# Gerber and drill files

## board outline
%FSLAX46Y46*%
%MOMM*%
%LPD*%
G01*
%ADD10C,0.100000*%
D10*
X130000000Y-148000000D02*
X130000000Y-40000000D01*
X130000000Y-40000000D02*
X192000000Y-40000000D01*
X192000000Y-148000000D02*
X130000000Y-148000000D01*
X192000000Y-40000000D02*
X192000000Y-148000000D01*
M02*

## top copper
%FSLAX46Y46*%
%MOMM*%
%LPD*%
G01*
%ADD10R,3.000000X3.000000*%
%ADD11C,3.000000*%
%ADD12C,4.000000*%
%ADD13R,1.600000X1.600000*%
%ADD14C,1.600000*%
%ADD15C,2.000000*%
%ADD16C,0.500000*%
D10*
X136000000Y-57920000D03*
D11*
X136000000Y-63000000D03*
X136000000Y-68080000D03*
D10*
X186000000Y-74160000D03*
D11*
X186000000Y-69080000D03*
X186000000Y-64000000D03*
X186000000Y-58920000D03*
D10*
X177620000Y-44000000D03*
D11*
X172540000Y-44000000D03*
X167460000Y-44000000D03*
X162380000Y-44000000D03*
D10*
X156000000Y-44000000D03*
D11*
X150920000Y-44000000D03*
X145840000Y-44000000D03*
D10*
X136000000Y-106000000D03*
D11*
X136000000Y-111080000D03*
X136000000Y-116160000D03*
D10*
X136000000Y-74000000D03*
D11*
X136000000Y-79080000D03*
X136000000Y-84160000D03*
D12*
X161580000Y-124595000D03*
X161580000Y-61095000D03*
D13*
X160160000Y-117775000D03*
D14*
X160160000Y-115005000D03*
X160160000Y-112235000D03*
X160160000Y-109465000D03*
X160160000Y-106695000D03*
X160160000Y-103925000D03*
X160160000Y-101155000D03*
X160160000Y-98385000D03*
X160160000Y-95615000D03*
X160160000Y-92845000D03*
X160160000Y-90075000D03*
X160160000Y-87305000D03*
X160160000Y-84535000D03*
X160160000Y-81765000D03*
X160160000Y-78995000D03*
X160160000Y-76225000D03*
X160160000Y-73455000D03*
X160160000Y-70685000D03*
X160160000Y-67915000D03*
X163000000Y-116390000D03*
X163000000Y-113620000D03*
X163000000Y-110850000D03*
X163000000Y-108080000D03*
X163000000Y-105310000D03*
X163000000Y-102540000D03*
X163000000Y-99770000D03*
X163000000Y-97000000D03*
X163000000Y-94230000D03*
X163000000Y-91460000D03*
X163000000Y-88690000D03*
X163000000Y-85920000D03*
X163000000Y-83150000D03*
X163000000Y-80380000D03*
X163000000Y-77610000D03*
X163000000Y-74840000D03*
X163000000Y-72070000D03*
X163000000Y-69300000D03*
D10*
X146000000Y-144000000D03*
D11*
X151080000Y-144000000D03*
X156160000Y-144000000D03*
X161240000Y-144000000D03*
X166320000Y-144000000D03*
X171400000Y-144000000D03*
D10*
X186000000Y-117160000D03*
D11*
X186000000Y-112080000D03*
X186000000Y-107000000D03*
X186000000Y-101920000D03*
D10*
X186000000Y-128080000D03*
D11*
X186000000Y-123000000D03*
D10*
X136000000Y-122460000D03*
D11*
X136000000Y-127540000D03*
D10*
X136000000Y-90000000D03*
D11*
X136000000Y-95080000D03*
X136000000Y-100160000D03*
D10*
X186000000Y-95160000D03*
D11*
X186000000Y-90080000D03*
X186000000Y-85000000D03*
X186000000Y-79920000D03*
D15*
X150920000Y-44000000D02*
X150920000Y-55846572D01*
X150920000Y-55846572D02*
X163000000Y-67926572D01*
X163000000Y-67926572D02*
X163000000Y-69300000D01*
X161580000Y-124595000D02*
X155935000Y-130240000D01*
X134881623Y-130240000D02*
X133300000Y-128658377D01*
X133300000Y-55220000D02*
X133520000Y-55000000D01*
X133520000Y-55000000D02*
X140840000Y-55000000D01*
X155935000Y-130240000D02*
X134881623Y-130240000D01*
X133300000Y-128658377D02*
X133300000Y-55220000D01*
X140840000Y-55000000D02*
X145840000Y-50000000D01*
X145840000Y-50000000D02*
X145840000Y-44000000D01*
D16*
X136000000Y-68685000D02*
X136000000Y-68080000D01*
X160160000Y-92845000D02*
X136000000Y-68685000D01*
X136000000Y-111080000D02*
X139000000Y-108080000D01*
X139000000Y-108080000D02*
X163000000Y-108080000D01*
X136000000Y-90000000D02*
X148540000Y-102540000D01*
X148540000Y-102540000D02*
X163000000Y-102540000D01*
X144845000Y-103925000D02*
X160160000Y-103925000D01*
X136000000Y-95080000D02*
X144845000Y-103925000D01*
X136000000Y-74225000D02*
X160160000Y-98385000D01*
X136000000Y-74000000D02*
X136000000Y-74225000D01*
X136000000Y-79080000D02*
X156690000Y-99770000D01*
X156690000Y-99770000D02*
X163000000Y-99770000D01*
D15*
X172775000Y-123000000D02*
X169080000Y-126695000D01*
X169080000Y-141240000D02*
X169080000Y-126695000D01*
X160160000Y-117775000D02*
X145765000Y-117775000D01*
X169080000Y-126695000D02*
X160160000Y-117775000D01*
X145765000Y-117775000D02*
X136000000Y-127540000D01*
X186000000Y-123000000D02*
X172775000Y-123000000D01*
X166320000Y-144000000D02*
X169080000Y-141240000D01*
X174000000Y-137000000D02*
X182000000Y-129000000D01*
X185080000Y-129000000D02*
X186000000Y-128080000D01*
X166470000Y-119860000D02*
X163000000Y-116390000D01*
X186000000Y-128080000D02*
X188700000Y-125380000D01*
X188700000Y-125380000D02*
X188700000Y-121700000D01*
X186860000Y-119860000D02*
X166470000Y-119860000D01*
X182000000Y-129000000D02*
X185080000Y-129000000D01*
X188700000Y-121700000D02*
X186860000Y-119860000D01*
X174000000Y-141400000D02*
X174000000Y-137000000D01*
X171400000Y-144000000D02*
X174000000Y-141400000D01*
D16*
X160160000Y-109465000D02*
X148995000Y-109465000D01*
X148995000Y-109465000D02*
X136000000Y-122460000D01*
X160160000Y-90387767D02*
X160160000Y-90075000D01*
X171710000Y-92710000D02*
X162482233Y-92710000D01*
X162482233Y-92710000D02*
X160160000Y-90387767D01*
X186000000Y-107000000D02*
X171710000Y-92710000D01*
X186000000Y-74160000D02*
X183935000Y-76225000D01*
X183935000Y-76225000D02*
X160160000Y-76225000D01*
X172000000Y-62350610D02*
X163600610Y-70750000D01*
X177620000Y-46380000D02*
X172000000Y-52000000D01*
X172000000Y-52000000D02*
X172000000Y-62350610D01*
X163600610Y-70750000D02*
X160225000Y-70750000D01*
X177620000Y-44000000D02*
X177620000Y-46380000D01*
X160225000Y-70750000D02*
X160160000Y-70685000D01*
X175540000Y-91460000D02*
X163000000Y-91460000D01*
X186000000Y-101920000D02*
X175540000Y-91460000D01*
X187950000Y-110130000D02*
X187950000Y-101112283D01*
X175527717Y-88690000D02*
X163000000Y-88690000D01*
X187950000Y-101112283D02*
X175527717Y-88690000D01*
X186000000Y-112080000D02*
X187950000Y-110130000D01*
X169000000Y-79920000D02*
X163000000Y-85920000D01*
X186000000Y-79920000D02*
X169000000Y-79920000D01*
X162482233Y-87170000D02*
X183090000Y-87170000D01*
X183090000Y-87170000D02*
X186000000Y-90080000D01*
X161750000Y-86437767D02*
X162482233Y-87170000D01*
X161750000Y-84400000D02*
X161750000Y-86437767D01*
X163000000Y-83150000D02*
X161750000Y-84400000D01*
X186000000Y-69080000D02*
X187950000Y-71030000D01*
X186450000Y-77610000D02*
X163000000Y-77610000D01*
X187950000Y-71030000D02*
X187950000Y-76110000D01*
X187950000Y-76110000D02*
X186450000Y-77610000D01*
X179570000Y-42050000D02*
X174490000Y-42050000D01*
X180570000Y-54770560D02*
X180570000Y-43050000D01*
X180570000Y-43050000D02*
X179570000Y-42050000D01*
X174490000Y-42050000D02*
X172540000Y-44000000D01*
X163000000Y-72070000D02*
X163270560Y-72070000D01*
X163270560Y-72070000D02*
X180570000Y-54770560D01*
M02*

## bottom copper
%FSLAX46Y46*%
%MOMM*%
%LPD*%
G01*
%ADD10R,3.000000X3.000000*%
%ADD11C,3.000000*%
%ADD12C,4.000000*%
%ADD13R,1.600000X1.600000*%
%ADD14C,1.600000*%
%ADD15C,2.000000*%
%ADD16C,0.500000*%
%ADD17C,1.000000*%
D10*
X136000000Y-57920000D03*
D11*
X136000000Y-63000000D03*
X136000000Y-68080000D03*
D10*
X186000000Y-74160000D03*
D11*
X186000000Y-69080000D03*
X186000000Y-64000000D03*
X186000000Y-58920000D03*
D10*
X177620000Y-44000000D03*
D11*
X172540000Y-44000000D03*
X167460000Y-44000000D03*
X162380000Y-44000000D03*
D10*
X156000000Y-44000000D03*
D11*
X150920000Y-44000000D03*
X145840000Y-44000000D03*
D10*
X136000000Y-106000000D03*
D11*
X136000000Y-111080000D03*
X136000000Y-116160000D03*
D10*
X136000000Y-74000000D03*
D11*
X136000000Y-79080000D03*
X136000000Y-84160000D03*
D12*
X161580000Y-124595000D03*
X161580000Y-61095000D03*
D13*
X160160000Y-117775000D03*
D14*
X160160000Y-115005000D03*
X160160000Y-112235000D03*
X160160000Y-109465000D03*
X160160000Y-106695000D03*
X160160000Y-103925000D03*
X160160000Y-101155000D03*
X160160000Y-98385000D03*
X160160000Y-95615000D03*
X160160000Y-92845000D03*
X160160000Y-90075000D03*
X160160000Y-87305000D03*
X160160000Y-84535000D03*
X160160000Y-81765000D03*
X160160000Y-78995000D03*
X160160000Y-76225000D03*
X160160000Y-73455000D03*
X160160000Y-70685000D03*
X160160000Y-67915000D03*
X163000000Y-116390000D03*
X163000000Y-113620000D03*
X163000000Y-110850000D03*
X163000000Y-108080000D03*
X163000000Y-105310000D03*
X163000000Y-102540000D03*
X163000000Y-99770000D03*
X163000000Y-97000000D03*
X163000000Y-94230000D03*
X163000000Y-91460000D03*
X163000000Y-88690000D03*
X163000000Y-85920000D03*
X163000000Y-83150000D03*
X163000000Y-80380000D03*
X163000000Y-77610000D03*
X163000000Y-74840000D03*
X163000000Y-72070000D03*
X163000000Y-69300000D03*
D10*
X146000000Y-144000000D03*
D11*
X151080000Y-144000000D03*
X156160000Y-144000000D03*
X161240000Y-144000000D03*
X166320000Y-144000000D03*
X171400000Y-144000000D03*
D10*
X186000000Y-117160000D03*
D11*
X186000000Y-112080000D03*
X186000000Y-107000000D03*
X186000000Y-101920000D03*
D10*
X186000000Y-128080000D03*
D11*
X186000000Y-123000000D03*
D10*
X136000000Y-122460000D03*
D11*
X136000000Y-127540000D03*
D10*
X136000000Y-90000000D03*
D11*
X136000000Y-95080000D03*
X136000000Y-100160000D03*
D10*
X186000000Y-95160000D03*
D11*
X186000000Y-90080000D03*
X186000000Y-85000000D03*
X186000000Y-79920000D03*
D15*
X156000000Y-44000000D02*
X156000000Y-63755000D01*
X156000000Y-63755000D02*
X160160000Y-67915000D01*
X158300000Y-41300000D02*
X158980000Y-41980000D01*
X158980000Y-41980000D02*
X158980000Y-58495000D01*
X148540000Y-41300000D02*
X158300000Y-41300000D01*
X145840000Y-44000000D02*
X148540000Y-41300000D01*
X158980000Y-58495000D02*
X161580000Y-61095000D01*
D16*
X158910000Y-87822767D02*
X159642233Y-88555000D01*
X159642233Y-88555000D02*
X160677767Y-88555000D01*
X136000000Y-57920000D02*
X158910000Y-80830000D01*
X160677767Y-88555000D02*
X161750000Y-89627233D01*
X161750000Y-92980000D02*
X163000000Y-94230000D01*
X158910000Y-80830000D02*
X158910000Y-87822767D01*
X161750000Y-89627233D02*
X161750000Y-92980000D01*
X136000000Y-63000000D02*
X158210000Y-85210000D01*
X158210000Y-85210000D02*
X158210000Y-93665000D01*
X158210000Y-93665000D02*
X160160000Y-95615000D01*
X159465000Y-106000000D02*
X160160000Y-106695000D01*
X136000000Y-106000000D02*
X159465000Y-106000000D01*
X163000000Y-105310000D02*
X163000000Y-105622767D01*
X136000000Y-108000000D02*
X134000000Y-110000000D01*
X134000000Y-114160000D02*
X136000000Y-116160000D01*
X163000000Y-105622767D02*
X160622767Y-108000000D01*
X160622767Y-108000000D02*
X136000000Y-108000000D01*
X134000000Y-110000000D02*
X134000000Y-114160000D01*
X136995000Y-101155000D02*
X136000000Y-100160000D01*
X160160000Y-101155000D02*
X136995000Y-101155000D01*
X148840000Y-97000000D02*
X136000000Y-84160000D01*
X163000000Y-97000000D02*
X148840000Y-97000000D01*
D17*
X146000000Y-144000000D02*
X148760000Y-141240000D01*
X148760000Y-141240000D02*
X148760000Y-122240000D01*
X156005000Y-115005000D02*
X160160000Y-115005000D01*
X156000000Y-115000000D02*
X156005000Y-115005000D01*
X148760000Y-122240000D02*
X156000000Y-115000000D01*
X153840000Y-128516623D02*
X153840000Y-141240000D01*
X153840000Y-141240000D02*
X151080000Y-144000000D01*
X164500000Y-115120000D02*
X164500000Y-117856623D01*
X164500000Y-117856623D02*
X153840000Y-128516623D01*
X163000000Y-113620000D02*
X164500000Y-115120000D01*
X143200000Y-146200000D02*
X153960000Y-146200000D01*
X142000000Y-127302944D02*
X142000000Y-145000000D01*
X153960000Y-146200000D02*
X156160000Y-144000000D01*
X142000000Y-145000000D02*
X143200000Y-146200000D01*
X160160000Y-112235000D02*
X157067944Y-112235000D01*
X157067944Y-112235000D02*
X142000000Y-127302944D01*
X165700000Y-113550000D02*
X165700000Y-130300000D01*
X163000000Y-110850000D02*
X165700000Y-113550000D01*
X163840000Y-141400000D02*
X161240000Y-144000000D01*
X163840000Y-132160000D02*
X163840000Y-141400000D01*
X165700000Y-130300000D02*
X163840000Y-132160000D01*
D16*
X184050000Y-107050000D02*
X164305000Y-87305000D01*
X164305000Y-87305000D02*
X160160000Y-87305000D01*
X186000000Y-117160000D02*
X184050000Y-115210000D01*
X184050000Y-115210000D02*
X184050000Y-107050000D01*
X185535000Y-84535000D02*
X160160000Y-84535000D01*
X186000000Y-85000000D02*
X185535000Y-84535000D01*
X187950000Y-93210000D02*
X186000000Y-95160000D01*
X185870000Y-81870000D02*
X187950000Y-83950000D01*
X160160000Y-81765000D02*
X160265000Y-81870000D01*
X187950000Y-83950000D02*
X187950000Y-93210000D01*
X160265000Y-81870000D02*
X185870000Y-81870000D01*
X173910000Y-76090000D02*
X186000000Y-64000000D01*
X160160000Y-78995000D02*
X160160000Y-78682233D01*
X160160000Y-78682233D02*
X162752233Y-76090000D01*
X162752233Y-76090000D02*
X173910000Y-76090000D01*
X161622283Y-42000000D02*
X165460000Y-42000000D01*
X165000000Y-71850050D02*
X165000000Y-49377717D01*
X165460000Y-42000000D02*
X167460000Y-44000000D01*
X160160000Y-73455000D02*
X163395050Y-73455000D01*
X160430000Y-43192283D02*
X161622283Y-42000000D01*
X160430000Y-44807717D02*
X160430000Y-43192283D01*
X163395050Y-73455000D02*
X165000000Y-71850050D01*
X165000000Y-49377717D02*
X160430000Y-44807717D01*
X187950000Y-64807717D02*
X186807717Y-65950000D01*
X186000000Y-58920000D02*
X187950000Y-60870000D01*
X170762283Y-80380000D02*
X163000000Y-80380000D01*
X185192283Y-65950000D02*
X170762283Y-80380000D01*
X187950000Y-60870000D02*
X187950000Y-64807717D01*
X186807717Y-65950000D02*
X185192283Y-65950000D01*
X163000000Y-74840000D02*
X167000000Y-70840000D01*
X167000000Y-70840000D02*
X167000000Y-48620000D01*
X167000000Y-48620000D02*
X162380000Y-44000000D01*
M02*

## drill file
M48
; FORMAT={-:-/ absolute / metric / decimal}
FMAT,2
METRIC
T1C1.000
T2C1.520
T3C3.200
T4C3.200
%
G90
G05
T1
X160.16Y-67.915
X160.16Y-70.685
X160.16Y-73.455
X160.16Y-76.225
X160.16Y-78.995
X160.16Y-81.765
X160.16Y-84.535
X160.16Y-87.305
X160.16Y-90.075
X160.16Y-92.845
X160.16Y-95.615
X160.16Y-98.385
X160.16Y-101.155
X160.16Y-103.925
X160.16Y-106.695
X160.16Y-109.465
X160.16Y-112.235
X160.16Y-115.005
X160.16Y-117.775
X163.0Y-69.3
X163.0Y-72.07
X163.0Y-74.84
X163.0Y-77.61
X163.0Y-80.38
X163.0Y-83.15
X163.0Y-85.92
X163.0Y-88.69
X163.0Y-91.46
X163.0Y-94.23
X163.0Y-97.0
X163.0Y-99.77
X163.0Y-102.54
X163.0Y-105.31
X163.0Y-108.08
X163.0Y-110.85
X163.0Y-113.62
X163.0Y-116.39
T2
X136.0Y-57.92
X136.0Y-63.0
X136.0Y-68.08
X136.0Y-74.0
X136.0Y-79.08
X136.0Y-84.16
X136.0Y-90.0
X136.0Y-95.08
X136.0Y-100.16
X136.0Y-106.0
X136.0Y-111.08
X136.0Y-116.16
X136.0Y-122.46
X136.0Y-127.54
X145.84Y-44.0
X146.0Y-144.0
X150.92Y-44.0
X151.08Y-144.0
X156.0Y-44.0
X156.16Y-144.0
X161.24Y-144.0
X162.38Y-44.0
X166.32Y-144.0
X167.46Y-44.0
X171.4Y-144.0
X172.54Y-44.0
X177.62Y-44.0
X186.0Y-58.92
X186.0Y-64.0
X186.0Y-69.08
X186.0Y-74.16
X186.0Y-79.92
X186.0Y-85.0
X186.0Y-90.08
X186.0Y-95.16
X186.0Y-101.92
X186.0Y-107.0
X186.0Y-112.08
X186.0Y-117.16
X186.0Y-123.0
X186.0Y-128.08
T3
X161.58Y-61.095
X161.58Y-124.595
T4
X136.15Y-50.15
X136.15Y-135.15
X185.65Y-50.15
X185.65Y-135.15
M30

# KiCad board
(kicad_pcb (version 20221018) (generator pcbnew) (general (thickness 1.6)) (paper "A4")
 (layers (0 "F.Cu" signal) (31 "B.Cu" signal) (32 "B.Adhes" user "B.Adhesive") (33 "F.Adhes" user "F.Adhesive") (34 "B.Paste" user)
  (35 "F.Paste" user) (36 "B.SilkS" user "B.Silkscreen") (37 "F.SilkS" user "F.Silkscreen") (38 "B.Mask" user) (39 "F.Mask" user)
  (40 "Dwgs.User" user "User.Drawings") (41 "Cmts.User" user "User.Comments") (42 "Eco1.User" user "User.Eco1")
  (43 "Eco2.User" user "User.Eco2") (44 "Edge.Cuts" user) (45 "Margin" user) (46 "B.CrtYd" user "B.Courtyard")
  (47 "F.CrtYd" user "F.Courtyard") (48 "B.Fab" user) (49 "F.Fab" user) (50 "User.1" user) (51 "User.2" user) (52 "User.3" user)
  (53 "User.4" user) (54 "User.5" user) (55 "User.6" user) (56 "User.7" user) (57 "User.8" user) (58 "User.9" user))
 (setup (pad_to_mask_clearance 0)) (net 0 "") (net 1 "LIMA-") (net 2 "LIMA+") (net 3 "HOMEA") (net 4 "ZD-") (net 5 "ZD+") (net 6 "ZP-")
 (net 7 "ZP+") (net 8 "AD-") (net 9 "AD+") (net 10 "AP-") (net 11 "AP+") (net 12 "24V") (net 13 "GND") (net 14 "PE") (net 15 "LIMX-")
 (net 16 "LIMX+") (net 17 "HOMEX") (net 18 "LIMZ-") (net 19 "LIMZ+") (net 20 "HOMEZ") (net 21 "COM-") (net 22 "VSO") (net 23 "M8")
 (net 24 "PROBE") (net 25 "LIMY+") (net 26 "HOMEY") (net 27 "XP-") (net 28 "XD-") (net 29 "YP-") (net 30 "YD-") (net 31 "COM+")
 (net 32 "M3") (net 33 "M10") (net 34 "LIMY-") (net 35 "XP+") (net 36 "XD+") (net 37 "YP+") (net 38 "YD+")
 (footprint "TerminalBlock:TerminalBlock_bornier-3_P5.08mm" (layer "F.Cu") (at 136 57.92 -90)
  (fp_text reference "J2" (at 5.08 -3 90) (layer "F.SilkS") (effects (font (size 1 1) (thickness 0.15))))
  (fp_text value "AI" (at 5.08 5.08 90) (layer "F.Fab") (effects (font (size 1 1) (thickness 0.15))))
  (pad "1" thru_hole rect (at 0 0 270) (size 3 3) (drill 1.52) (layers "*.Cu" "*.Mask") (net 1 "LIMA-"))
  (pad "2" thru_hole circle (at 5.08 0 270) (size 3 3) (drill 1.52) (layers "*.Cu" "*.Mask") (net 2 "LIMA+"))
  (pad "3" thru_hole circle (at 10.16 0 270) (size 3 3) (drill 1.52) (layers "*.Cu" "*.Mask") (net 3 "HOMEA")))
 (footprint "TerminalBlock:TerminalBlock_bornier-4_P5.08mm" (layer "F.Cu") (at 186 74.16 90)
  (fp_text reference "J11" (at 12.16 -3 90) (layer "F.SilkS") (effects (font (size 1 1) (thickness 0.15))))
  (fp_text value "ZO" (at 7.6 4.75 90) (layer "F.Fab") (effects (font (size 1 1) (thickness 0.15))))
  (pad "1" thru_hole rect (at 0 0 90) (size 3 3) (drill 1.52) (layers "*.Cu" "*.Mask") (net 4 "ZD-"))
  (pad "2" thru_hole circle (at 5.08 0 90) (size 3 3) (drill 1.52) (layers "*.Cu" "*.Mask") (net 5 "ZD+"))
  (pad "3" thru_hole circle (at 10.16 0 90) (size 3 3) (drill 1.52) (layers "*.Cu" "*.Mask") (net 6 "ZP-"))
  (pad "4" thru_hole circle (at 15.24 0 90) (size 3 3) (drill 1.52) (layers "*.Cu" "*.Mask") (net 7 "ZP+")))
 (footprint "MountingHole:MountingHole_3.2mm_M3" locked (layer "F.Cu") (at 185.65 50.15)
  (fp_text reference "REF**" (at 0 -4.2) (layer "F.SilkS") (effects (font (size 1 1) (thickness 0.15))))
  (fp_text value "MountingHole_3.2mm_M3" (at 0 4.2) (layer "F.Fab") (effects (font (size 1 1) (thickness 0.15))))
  (pad "" np_thru_hole circle locked (at 0 0) (size 3.2 3.2) (drill 3.2) (layers "*.Cu" "*.Mask")))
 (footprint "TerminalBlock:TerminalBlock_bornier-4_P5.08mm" (layer "F.Cu") (at 177.62 44 180)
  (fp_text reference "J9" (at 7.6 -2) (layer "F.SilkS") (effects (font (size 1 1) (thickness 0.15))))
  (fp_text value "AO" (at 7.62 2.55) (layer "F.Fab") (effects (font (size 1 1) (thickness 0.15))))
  (pad "1" thru_hole rect (at 0 0 180) (size 3 3) (drill 1.52) (layers "*.Cu" "*.Mask") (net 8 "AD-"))
  (pad "2" thru_hole circle (at 5.08 0 180) (size 3 3) (drill 1.52) (layers "*.Cu" "*.Mask") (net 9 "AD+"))
  (pad "3" thru_hole circle (at 10.16 0 180) (size 3 3) (drill 1.52) (layers "*.Cu" "*.Mask") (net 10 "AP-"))
  (pad "4" thru_hole circle (at 15.24 0 180) (size 3 3) (drill 1.52) (layers "*.Cu" "*.Mask") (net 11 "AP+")))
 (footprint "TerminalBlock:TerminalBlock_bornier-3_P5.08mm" (layer "F.Cu") (at 156 44 180)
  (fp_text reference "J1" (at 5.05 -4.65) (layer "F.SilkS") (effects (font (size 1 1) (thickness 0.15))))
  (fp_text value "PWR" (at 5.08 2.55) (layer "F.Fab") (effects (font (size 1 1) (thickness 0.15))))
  (pad "1" thru_hole rect (at 0 0 180) (size 3 3) (drill 1.52) (layers "*.Cu" "*.Mask") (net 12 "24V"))
  (pad "2" thru_hole circle (at 5.08 0 180) (size 3 3) (drill 1.52) (layers "*.Cu" "*.Mask") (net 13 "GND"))
  (pad "3" thru_hole circle (at 10.16 0 180) (size 3 3) (drill 1.52) (layers "*.Cu" "*.Mask") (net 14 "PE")))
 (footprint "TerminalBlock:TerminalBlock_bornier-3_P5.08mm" (layer "F.Cu") (at 136 106 -90)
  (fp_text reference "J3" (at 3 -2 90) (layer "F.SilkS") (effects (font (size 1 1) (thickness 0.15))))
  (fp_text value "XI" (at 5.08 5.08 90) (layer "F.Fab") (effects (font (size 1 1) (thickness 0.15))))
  (pad "1" thru_hole rect (at 0 0 270) (size 3 3) (drill 1.52) (layers "*.Cu" "*.Mask") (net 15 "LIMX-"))
  (pad "2" thru_hole circle (at 5.08 0 270) (size 3 3) (drill 1.52) (layers "*.Cu" "*.Mask") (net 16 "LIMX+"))
  (pad "3" thru_hole circle (at 10.16 0 270) (size 3 3) (drill 1.52) (layers "*.Cu" "*.Mask") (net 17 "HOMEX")))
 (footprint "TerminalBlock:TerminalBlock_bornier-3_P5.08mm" (layer "F.Cu") (at 136 74 -90)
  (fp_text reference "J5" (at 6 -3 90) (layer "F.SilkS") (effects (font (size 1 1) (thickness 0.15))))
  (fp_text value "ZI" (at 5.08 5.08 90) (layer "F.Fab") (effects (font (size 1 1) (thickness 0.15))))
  (pad "1" thru_hole rect (at 0 0 270) (size 3 3) (drill 1.52) (layers "*.Cu" "*.Mask") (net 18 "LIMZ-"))
  (pad "2" thru_hole circle (at 5.08 0 270) (size 3 3) (drill 1.52) (layers "*.Cu" "*.Mask") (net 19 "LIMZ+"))
  (pad "3" thru_hole circle (at 10.16 0 270) (size 3 3) (drill 1.52) (layers "*.Cu" "*.Mask") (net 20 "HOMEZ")))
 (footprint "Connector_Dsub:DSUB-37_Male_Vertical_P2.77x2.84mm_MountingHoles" (layer "F.Cu") (at 160.16 117.775 90)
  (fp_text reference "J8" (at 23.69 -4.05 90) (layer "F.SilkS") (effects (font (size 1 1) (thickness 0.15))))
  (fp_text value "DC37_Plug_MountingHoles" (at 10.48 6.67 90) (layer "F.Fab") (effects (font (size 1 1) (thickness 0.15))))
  (pad "0" thru_hole circle (at -6.82 1.42 90) (size 4 4) (drill 3.2) (layers "*.Cu" "*.Mask") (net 14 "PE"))
  (pad "0" thru_hole circle (at 56.68 1.42 90) (size 4 4) (drill 3.2) (layers "*.Cu" "*.Mask") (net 14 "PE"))
  (pad "1" thru_hole rect (at 0 0 90) (size 1.6 1.6) (drill 1) (layers "*.Cu" "*.Mask") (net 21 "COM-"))
  (pad "2" thru_hole circle (at 2.77 0 90) (size 1.6 1.6) (drill 1) (layers "*.Cu" "*.Mask") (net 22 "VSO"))
  (pad "3" thru_hole circle (at 5.54 0 90) (size 1.6 1.6) (drill 1) (layers "*.Cu" "*.Mask") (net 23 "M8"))
  (pad "4" thru_hole circle (at 8.31 0 90) (size 1.6 1.6) (drill 1) (layers "*.Cu" "*.Mask") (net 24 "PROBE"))
  (pad "5" thru_hole circle (at 11.08 0 90) (size 1.6 1.6) (drill 1) (layers "*.Cu" "*.Mask") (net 15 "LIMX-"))
  (pad "6" thru_hole circle (at 13.85 0 90) (size 1.6 1.6) (drill 1) (layers "*.Cu" "*.Mask") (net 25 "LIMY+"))
  (pad "7" thru_hole circle (at 16.62 0 90) (size 1.6 1.6) (drill 1) (layers "*.Cu" "*.Mask") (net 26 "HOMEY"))
  (pad "8" thru_hole circle (at 19.39 0 90) (size 1.6 1.6) (drill 1) (layers "*.Cu" "*.Mask") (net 18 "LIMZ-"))
  (pad "9" thru_hole circle (at 22.16 0 90) (size 1.6 1.6) (drill 1) (layers "*.Cu" "*.Mask") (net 2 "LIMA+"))
  (pad "10" thru_hole circle (at 24.93 0 90) (size 1.6 1.6) (drill 1) (layers "*.Cu" "*.Mask") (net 3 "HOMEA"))
  (pad "11" thru_hole circle (at 27.7 0 90) (size 1.6 1.6) (drill 1) (layers "*.Cu" "*.Mask") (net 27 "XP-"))
  (pad "12" thru_hole circle (at 30.47 0 90) (size 1.6 1.6) (drill 1) (layers "*.Cu" "*.Mask") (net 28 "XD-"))
  (pad "13" thru_hole circle (at 33.24 0 90) (size 1.6 1.6) (drill 1) (layers "*.Cu" "*.Mask") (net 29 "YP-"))
  (pad "14" thru_hole circle (at 36.01 0 90) (size 1.6 1.6) (drill 1) (layers "*.Cu" "*.Mask") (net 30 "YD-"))
  (pad "15" thru_hole circle (at 38.78 0 90) (size 1.6 1.6) (drill 1) (layers "*.Cu" "*.Mask") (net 6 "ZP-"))
  (pad "16" thru_hole circle (at 41.55 0 90) (size 1.6 1.6) (drill 1) (layers "*.Cu" "*.Mask") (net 4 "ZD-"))
  (pad "17" thru_hole circle (at 44.32 0 90) (size 1.6 1.6) (drill 1) (layers "*.Cu" "*.Mask") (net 10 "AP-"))
  (pad "18" thru_hole circle (at 47.09 0 90) (size 1.6 1.6) (drill 1) (layers "*.Cu" "*.Mask") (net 8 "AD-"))
  (pad "19" thru_hole circle (at 49.86 0 90) (size 1.6 1.6) (drill 1) (layers "*.Cu" "*.Mask") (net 12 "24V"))
  (pad "20" thru_hole circle (at 1.385 2.84 90) (size 1.6 1.6) (drill 1) (layers "*.Cu" "*.Mask") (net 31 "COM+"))
  (pad "21" thru_hole circle (at 4.155 2.84 90) (size 1.6 1.6) (drill 1) (layers "*.Cu" "*.Mask") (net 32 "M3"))
  (pad "22" thru_hole circle (at 6.925 2.84 90) (size 1.6 1.6) (drill 1) (layers "*.Cu" "*.Mask") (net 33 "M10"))
  (pad "23" thru_hole circle (at 9.695 2.84 90) (size 1.6 1.6) (drill 1) (layers "*.Cu" "*.Mask") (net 16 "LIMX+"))
  (pad "24" thru_hole circle (at 12.465 2.84 90) (size 1.6 1.6) (drill 1) (layers "*.Cu" "*.Mask") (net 17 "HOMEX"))
  (pad "25" thru_hole circle (at 15.235 2.84 90) (size 1.6 1.6) (drill 1) (layers "*.Cu" "*.Mask") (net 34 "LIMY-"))
  (pad "26" thru_hole circle (at 18.005 2.84 90) (size 1.6 1.6) (drill 1) (layers "*.Cu" "*.Mask") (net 19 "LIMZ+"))
  (pad "27" thru_hole circle (at 20.775 2.84 90) (size 1.6 1.6) (drill 1) (layers "*.Cu" "*.Mask") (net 20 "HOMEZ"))
  (pad "28" thru_hole circle (at 23.545 2.84 90) (size 1.6 1.6) (drill 1) (layers "*.Cu" "*.Mask") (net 1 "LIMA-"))
  (pad "29" thru_hole circle (at 26.315 2.84 90) (size 1.6 1.6) (drill 1) (layers "*.Cu" "*.Mask") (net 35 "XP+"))
  (pad "30" thru_hole circle (at 29.085 2.84 90) (size 1.6 1.6) (drill 1) (layers "*.Cu" "*.Mask") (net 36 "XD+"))
  (pad "31" thru_hole circle (at 31.855 2.84 90) (size 1.6 1.6) (drill 1) (layers "*.Cu" "*.Mask") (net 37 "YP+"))
  (pad "32" thru_hole circle (at 34.625 2.84 90) (size 1.6 1.6) (drill 1) (layers "*.Cu" "*.Mask") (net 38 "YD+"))
  (pad "33" thru_hole circle (at 37.395 2.84 90) (size 1.6 1.6) (drill 1) (layers "*.Cu" "*.Mask") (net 7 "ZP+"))
  (pad "34" thru_hole circle (at 40.165 2.84 90) (size 1.6 1.6) (drill 1) (layers "*.Cu" "*.Mask") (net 5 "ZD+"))
  (pad "35" thru_hole circle (at 42.935 2.84 90) (size 1.6 1.6) (drill 1) (layers "*.Cu" "*.Mask") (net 11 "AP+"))
  (pad "36" thru_hole circle (at 45.705 2.84 90) (size 1.6 1.6) (drill 1) (layers "*.Cu" "*.Mask") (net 9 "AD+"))
  (pad "37" thru_hole circle (at 48.475 2.84 90) (size 1.6 1.6) (drill 1) (layers "*.Cu" "*.Mask") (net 13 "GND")))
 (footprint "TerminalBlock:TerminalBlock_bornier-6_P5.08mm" (layer "F.Cu") (at 146 144)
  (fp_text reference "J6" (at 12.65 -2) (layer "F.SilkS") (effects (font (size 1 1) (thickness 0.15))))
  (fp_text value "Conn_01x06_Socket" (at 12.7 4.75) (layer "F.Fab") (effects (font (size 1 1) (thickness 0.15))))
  (pad "1" thru_hole rect (at 0 0) (size 3 3) (drill 1.52) (layers "*.Cu" "*.Mask") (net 22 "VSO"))
  (pad "2" thru_hole circle (at 5.08 0) (size 3 3) (drill 1.52) (layers "*.Cu" "*.Mask") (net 32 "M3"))
  (pad "3" thru_hole circle (at 10.16 0) (size 3 3) (drill 1.52) (layers "*.Cu" "*.Mask") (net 23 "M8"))
  (pad "4" thru_hole circle (at 15.24 0) (size 3 3) (drill 1.52) (layers "*.Cu" "*.Mask") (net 33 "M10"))
  (pad "5" thru_hole circle (at 20.32 0) (size 3 3) (drill 1.52) (layers "*.Cu" "*.Mask") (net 21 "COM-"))
  (pad "6" thru_hole circle (at 25.4 0) (size 3 3) (drill 1.52) (layers "*.Cu" "*.Mask") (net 31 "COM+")))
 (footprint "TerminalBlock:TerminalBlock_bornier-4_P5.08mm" (layer "F.Cu") (at 186 117.16 90)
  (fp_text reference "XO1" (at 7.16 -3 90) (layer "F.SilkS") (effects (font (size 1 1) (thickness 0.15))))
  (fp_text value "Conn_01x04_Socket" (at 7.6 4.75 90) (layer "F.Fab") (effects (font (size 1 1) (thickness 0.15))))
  (pad "1" thru_hole rect (at 0 0 90) (size 3 3) (drill 1.52) (layers "*.Cu" "*.Mask") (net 28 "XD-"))
  (pad "2" thru_hole circle (at 5.08 0 90) (size 3 3) (drill 1.52) (layers "*.Cu" "*.Mask") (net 36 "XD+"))
  (pad "3" thru_hole circle (at 10.16 0 90) (size 3 3) (drill 1.52) (layers "*.Cu" "*.Mask") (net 27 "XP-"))
  (pad "4" thru_hole circle (at 15.24 0 90) (size 3 3) (drill 1.52) (layers "*.Cu" "*.Mask") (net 35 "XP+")))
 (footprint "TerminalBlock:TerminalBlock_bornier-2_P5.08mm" (layer "F.Cu") (at 186 128.08 90)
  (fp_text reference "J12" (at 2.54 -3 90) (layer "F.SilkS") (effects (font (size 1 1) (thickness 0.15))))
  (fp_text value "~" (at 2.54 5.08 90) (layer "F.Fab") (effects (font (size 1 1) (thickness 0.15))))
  (pad "1" thru_hole rect (at 0 0 90) (size 3 3) (drill 1.52) (layers "*.Cu" "*.Mask") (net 31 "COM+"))
  (pad "2" thru_hole circle (at 5.08 0 90) (size 3 3) (drill 1.52) (layers "*.Cu" "*.Mask") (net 21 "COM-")))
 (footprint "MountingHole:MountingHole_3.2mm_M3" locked (layer "F.Cu") (at 185.65 135.15)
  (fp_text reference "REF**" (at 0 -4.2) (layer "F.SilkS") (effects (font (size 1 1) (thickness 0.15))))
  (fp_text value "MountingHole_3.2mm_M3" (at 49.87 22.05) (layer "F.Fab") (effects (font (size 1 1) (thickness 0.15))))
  (pad "" np_thru_hole circle locked (at 0 0) (size 3.2 3.2) (drill 3.2) (layers "*.Cu" "*.Mask")))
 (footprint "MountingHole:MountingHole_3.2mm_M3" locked (layer "F.Cu") (at 136.15 50.15)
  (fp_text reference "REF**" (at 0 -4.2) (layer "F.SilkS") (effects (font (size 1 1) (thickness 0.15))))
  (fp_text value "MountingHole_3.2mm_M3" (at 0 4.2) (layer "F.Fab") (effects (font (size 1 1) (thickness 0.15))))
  (pad "" np_thru_hole circle locked (at 0 0) (size 3.2 3.2) (drill 3.2) (layers "*.Cu" "*.Mask")))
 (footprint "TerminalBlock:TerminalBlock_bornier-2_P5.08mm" (layer "F.Cu") (at 136 122.46 -90)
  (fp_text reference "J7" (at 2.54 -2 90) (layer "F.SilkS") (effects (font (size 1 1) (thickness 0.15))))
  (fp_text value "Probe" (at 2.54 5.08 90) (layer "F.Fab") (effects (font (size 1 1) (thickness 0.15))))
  (pad "1" thru_hole rect (at 0 0 270) (size 3 3) (drill 1.52) (layers "*.Cu" "*.Mask") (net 24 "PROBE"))
  (pad "2" thru_hole circle (at 5.08 0 270) (size 3 3) (drill 1.52) (layers "*.Cu" "*.Mask") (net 21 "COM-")))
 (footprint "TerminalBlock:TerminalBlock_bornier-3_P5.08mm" (layer "F.Cu") (at 136 90 -90)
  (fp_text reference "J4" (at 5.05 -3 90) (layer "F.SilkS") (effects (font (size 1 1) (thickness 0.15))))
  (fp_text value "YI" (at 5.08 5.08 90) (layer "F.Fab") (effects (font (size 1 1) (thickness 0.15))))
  (pad "1" thru_hole rect (at 0 0 270) (size 3 3) (drill 1.52) (layers "*.Cu" "*.Mask") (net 34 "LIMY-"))
  (pad "2" thru_hole circle (at 5.08 0 270) (size 3 3) (drill 1.52) (layers "*.Cu" "*.Mask") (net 25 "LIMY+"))
  (pad "3" thru_hole circle (at 10.16 0 270) (size 3 3) (drill 1.52) (layers "*.Cu" "*.Mask") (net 26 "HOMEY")))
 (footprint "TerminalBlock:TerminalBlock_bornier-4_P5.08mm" (layer "F.Cu") (at 186 95.16 90)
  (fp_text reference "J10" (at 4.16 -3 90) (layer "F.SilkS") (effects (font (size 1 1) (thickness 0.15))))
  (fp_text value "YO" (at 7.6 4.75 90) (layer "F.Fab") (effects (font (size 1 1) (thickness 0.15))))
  (pad "1" thru_hole rect (at 0 0 90) (size 3 3) (drill 1.52) (layers "*.Cu" "*.Mask") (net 30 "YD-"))
  (pad "2" thru_hole circle (at 5.08 0 90) (size 3 3) (drill 1.52) (layers "*.Cu" "*.Mask") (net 38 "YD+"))
  (pad "3" thru_hole circle (at 10.16 0 90) (size 3 3) (drill 1.52) (layers "*.Cu" "*.Mask") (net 29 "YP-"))
  (pad "4" thru_hole circle (at 15.24 0 90) (size 3 3) (drill 1.52) (layers "*.Cu" "*.Mask") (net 37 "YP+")))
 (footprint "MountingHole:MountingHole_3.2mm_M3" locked (layer "F.Cu") (at 136.15 135.15)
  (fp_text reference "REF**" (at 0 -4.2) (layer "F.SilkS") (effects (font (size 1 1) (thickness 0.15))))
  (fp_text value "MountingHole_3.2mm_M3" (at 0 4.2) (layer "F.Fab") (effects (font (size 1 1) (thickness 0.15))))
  (pad "" np_thru_hole circle locked (at 0 0) (size 3.2 3.2) (drill 3.2) (layers "*.Cu" "*.Mask")))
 (gr_line (start 130 148) (end 130 40) (stroke (width 0.1) (type default)) (layer "Edge.Cuts"))
 (gr_line (start 130 40) (end 192 40) (stroke (width 0.1) (type default)) (layer "Edge.Cuts"))
 (gr_line (start 192 148) (end 130 148) (stroke (width 0.1) (type default)) (layer "Edge.Cuts"))
 (gr_line (start 192 40) (end 192 148) (stroke (width 0.1) (type default)) (layer "Edge.Cuts"))
 (segment (start 156 44) (end 156 63.755) (width 2) (layer "B.Cu") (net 12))
 (segment (start 156 63.755) (end 160.16 67.915) (width 2) (layer "B.Cu") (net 12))
 (segment (start 150.92 44) (end 150.92 55.846572) (width 2) (layer "F.Cu") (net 13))
 (segment (start 150.92 55.846572) (end 163 67.926572) (width 2) (layer "F.Cu") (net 13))
 (segment (start 163 67.926572) (end 163 69.3) (width 2) (layer "F.Cu") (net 13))
 (segment (start 161.58 124.595) (end 155.935 130.24) (width 2) (layer "F.Cu") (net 14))
 (segment (start 134.881623 130.24) (end 133.3 128.658377) (width 2) (layer "F.Cu") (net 14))
 (segment (start 133.3 55.22) (end 133.52 55) (width 2) (layer "F.Cu") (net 14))
 (segment (start 133.52 55) (end 140.84 55) (width 2) (layer "F.Cu") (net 14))
 (segment (start 155.935 130.24) (end 134.881623 130.24) (width 2) (layer "F.Cu") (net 14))
 (segment (start 133.3 128.658377) (end 133.3 55.22) (width 2) (layer "F.Cu") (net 14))
 (segment (start 140.84 55) (end 145.84 50) (width 2) (layer "F.Cu") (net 14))
 (segment (start 145.84 50) (end 145.84 44) (width 2) (layer "F.Cu") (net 14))
 (segment (start 158.3 41.3) (end 158.98 41.98) (width 2) (layer "B.Cu") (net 14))
 (segment (start 158.98 41.98) (end 158.98 58.495) (width 2) (layer "B.Cu") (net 14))
 (segment (start 148.54 41.3) (end 158.3 41.3) (width 2) (layer "B.Cu") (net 14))
 (segment (start 145.84 44) (end 148.54 41.3) (width 2) (layer "B.Cu") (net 14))
 (segment (start 158.98 58.495) (end 161.58 61.095) (width 2) (layer "B.Cu") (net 14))
 (segment (start 158.91 87.822767) (end 159.642233 88.555) (width 0.5) (layer "B.Cu") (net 1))
 (segment (start 159.642233 88.555) (end 160.677767 88.555) (width 0.5) (layer "B.Cu") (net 1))
 (segment (start 136 57.92) (end 158.91 80.83) (width 0.5) (layer "B.Cu") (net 1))
 (segment (start 160.677767 88.555) (end 161.75 89.627233) (width 0.5) (layer "B.Cu") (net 1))
 (segment (start 161.75 92.98) (end 163 94.23) (width 0.5) (layer "B.Cu") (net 1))
 (segment (start 158.91 80.83) (end 158.91 87.822767) (width 0.5) (layer "B.Cu") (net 1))
 (segment (start 161.75 89.627233) (end 161.75 92.98) (width 0.5) (layer "B.Cu") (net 1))
 (segment (start 136 63) (end 158.21 85.21) (width 0.5) (layer "B.Cu") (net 2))
 (segment (start 158.21 85.21) (end 158.21 93.665) (width 0.5) (layer "B.Cu") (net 2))
 (segment (start 158.21 93.665) (end 160.16 95.615) (width 0.5) (layer "B.Cu") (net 2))
 (segment (start 136 68.685) (end 136 68.08) (width 0.5) (layer "F.Cu") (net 3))
 (segment (start 160.16 92.845) (end 136 68.685) (width 0.5) (layer "F.Cu") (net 3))
 (segment (start 159.465 106) (end 160.16 106.695) (width 0.5) (layer "B.Cu") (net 15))
 (segment (start 136 106) (end 159.465 106) (width 0.5) (layer "B.Cu") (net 15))
 (segment (start 136 111.08) (end 139 108.08) (width 0.5) (layer "F.Cu") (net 16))
 (segment (start 139 108.08) (end 163 108.08) (width 0.5) (layer "F.Cu") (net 16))
 (segment (start 163 105.31) (end 163 105.622767) (width 0.5) (layer "B.Cu") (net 17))
 (segment (start 136 108) (end 134 110) (width 0.5) (layer "B.Cu") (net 17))
 (segment (start 134 114.16) (end 136 116.16) (width 0.5) (layer "B.Cu") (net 17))
 (segment (start 163 105.622767) (end 160.622767 108) (width 0.5) (layer "B.Cu") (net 17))
 (segment (start 160.622767 108) (end 136 108) (width 0.5) (layer "B.Cu") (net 17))
 (segment (start 134 110) (end 134 114.16) (width 0.5) (layer "B.Cu") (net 17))
 (segment (start 136 90) (end 148.54 102.54) (width 0.5) (layer "F.Cu") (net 34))
 (segment (start 148.54 102.54) (end 163 102.54) (width 0.5) (layer "F.Cu") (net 34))
 (segment (start 144.845 103.925) (end 160.16 103.925) (width 0.5) (layer "F.Cu") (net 25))
 (segment (start 136 95.08) (end 144.845 103.925) (width 0.5) (layer "F.Cu") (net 25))
 (segment (start 136.995 101.155) (end 136 100.16) (width 0.5) (layer "B.Cu") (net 26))
 (segment (start 160.16 101.155) (end 136.995 101.155) (width 0.5) (layer "B.Cu") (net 26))
 (segment (start 136 74.225) (end 160.16 98.385) (width 0.5) (layer "F.Cu") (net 18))
 (segment (start 136 74) (end 136 74.225) (width 0.5) (layer "F.Cu") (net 18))
 (segment (start 136 79.08) (end 156.69 99.77) (width 0.5) (layer "F.Cu") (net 19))
 (segment (start 156.69 99.77) (end 163 99.77) (width 0.5) (layer "F.Cu") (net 19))
 (segment (start 148.84 97) (end 136 84.16) (width 0.5) (layer "B.Cu") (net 20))
 (segment (start 163 97) (end 148.84 97) (width 0.5) (layer "B.Cu") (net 20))
 (segment (start 146 144) (end 148.76 141.24) (width 1) (layer "B.Cu") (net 22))
 (segment (start 148.76 141.24) (end 148.76 122.24) (width 1) (layer "B.Cu") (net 22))
 (segment (start 156.005 115.005) (end 160.16 115.005) (width 1) (layer "B.Cu") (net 22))
 (segment (start 156 115) (end 156.005 115.005) (width 1) (layer "B.Cu") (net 22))
 (segment (start 148.76 122.24) (end 156 115) (width 1) (layer "B.Cu") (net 22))
 (segment (start 153.84 128.516623) (end 153.84 141.24) (width 1) (layer "B.Cu") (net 32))
 (segment (start 153.84 141.24) (end 151.08 144) (width 1) (layer "B.Cu") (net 32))
 (segment (start 164.5 115.12) (end 164.5 117.856623) (width 1) (layer "B.Cu") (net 32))
 (segment (start 164.5 117.856623) (end 153.84 128.516623) (width 1) (layer "B.Cu") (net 32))
 (segment (start 163 113.62) (end 164.5 115.12) (width 1) (layer "B.Cu") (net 32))
 (segment (start 143.2 146.2) (end 153.96 146.2) (width 1) (layer "B.Cu") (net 23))
 (segment (start 142 127.302944) (end 142 145) (width 1) (layer "B.Cu") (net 23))
 (segment (start 153.96 146.2) (end 156.16 144) (width 1) (layer "B.Cu") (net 23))
 (segment (start 142 145) (end 143.2 146.2) (width 1) (layer "B.Cu") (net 23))
 (segment (start 160.16 112.235) (end 157.067944 112.235) (width 1) (layer "B.Cu") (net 23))
 (segment (start 157.067944 112.235) (end 142 127.302944) (width 1) (layer "B.Cu") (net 23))
 (segment (start 165.7 113.55) (end 165.7 130.3) (width 1) (layer "B.Cu") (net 33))
 (segment (start 163 110.85) (end 165.7 113.55) (width 1) (layer "B.Cu") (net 33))
 (segment (start 163.84 141.4) (end 161.24 144) (width 1) (layer "B.Cu") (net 33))
 (segment (start 163.84 132.16) (end 163.84 141.4) (width 1) (layer "B.Cu") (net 33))
 (segment (start 165.7 130.3) (end 163.84 132.16) (width 1) (layer "B.Cu") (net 33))
 (segment (start 172.775 123) (end 169.08 126.695) (width 2) (layer "F.Cu") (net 21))
 (segment (start 169.08 141.24) (end 169.08 126.695) (width 2) (layer "F.Cu") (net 21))
 (segment (start 160.16 117.775) (end 145.765 117.775) (width 2) (layer "F.Cu") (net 21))
 (segment (start 169.08 126.695) (end 160.16 117.775) (width 2) (layer "F.Cu") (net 21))
 (segment (start 145.765 117.775) (end 136 127.54) (width 2) (layer "F.Cu") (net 21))
 (segment (start 186 123) (end 172.775 123) (width 2) (layer "F.Cu") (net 21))
 (segment (start 166.32 144) (end 169.08 141.24) (width 2) (layer "F.Cu") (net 21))
 (segment (start 174 137) (end 182 129) (width 2) (layer "F.Cu") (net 31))
 (segment (start 185.08 129) (end 186 128.08) (width 2) (layer "F.Cu") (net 31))
 (segment (start 166.47 119.86) (end 163 116.39) (width 2) (layer "F.Cu") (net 31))
 (segment (start 186 128.08) (end 188.7 125.38) (width 2) (layer "F.Cu") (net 31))
 (segment (start 188.7 125.38) (end 188.7 121.7) (width 2) (layer "F.Cu") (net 31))
 (segment (start 186.86 119.86) (end 166.47 119.86) (width 2) (layer "F.Cu") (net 31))
 (segment (start 182 129) (end 185.08 129) (width 2) (layer "F.Cu") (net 31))
 (segment (start 188.7 121.7) (end 186.86 119.86) (width 2) (layer "F.Cu") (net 31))
 (segment (start 174 141.4) (end 174 137) (width 2) (layer "F.Cu") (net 31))
 (segment (start 171.4 144) (end 174 141.4) (width 2) (layer "F.Cu") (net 31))
 (segment (start 160.16 109.465) (end 148.995 109.465) (width 0.5) (layer "F.Cu") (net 24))
 (segment (start 148.995 109.465) (end 136 122.46) (width 0.5) (layer "F.Cu") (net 24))
 (segment (start 160.16 90.387767) (end 160.16 90.075) (width 0.5) (layer "F.Cu") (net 27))
 (segment (start 171.71 92.71) (end 162.482233 92.71) (width 0.5) (layer "F.Cu") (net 27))
 (segment (start 162.482233 92.71) (end 160.16 90.387767) (width 0.5) (layer "F.Cu") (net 27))
 (segment (start 186 107) (end 171.71 92.71) (width 0.5) (layer "F.Cu") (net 27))
 (segment (start 184.05 107.05) (end 164.305 87.305) (width 0.5) (layer "B.Cu") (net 28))
 (segment (start 164.305 87.305) (end 160.16 87.305) (width 0.5) (layer "B.Cu") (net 28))
 (segment (start 186 117.16) (end 184.05 115.21) (width 0.5) (layer "B.Cu") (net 28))
 (segment (start 184.05 115.21) (end 184.05 107.05) (width 0.5) (layer "B.Cu") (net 28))
 (segment (start 185.535 84.535) (end 160.16 84.535) (width 0.5) (layer "B.Cu") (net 29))
 (segment (start 186 85) (end 185.535 84.535) (width 0.5) (layer "B.Cu") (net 29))
 (segment (start 187.95 93.21) (end 186 95.16) (width 0.5) (layer "B.Cu") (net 30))
 (segment (start 185.87 81.87) (end 187.95 83.95) (width 0.5) (layer "B.Cu") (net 30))
 (segment (start 160.16 81.765) (end 160.265 81.87) (width 0.5) (layer "B.Cu") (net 30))
 (segment (start 187.95 83.95) (end 187.95 93.21) (width 0.5) (layer "B.Cu") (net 30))
 (segment (start 160.265 81.87) (end 185.87 81.87) (width 0.5) (layer "B.Cu") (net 30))
 (segment (start 173.91 76.09) (end 186 64) (width 0.5) (layer "B.Cu") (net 6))
 (segment (start 160.16 78.995) (end 160.16 78.682233) (width 0.5) (layer "B.Cu") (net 6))
 (segment (start 160.16 78.682233) (end 162.752233 76.09) (width 0.5) (layer "B.Cu") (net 6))
 (segment (start 162.752233 76.09) (end 173.91 76.09) (width 0.5) (layer "B.Cu") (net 6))
 (segment (start 186 74.16) (end 183.935 76.225) (width 0.5) (layer "F.Cu") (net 4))
 (segment (start 183.935 76.225) (end 160.16 76.225) (width 0.5) (layer "F.Cu") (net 4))
 (segment (start 161.622283 42) (end 165.46 42) (width 0.5) (layer "B.Cu") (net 10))
 (segment (start 165 71.85005) (end 165 49.377717) (width 0.5) (layer "B.Cu") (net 10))
 (segment (start 165.46 42) (end 167.46 44) (width 0.5) (layer "B.Cu") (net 10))
 (segment (start 160.16 73.455) (end 163.39505 73.455) (width 0.5) (layer "B.Cu") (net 10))
 (segment (start 160.43 43.192283) (end 161.622283 42) (width 0.5) (layer "B.Cu") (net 10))
 (segment (start 160.43 44.807717) (end 160.43 43.192283) (width 0.5) (layer "B.Cu") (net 10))
 (segment (start 163.39505 73.455) (end 165 71.85005) (width 0.5) (layer "B.Cu") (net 10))
 (segment (start 165 49.377717) (end 160.43 44.807717) (width 0.5) (layer "B.Cu") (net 10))
 (segment (start 172 62.35061) (end 163.60061 70.75) (width 0.5) (layer "F.Cu") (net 8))
 (segment (start 177.62 46.38) (end 172 52) (width 0.5) (layer "F.Cu") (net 8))
 (segment (start 172 52) (end 172 62.35061) (width 0.5) (layer "F.Cu") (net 8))
 (segment (start 163.60061 70.75) (end 160.225 70.75) (width 0.5) (layer "F.Cu") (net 8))
 (segment (start 177.62 44) (end 177.62 46.38) (width 0.5) (layer "F.Cu") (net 8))
 (segment (start 160.225 70.75) (end 160.16 70.685) (width 0.5) (layer "F.Cu") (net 8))
 (segment (start 175.54 91.46) (end 163 91.46) (width 0.5) (layer "F.Cu") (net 35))
 (segment (start 186 101.92) (end 175.54 91.46) (width 0.5) (layer "F.Cu") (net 35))
 (segment (start 187.95 110.13) (end 187.95 101.112283) (width 0.5) (layer "F.Cu") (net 36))
 (segment (start 175.527717 88.69) (end 163 88.69) (width 0.5) (layer "F.Cu") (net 36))
 (segment (start 187.95 101.112283) (end 175.527717 88.69) (width 0.5) (layer "F.Cu") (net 36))
 (segment (start 186 112.08) (end 187.95 110.13) (width 0.5) (layer "F.Cu") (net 36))
 (segment (start 169 79.92) (end 163 85.92) (width 0.5) (layer "F.Cu") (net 37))
 (segment (start 186 79.92) (end 169 79.92) (width 0.5) (layer "F.Cu") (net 37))
 (segment (start 162.482233 87.17) (end 183.09 87.17) (width 0.5) (layer "F.Cu") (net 38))
 (segment (start 183.09 87.17) (end 186 90.08) (width 0.5) (layer "F.Cu") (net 38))
 (segment (start 161.75 86.437767) (end 162.482233 87.17) (width 0.5) (layer "F.Cu") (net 38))
 (segment (start 161.75 84.4) (end 161.75 86.437767) (width 0.5) (layer "F.Cu") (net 38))
 (segment (start 163 83.15) (end 161.75 84.4) (width 0.5) (layer "F.Cu") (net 38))
 (segment (start 187.95 64.807717) (end 186.807717 65.95) (width 0.5) (layer "B.Cu") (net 7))
 (segment (start 186 58.92) (end 187.95 60.87) (width 0.5) (layer "B.Cu") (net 7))
 (segment (start 170.762283 80.38) (end 163 80.38) (width 0.5) (layer "B.Cu") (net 7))
 (segment (start 185.192283 65.95) (end 170.762283 80.38) (width 0.5) (layer "B.Cu") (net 7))
 (segment (start 187.95 60.87) (end 187.95 64.807717) (width 0.5) (layer "B.Cu") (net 7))
 (segment (start 186.807717 65.95) (end 185.192283 65.95) (width 0.5) (layer "B.Cu") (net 7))
 (segment (start 186 69.08) (end 187.95 71.03) (width 0.5) (layer "F.Cu") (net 5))
 (segment (start 186.45 77.61) (end 163 77.61) (width 0.5) (layer "F.Cu") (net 5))
 (segment (start 187.95 71.03) (end 187.95 76.11) (width 0.5) (layer "F.Cu") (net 5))
 (segment (start 187.95 76.11) (end 186.45 77.61) (width 0.5) (layer "F.Cu") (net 5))
 (segment (start 163 74.84) (end 167 70.84) (width 0.5) (layer "B.Cu") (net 11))
 (segment (start 167 70.84) (end 167 48.62) (width 0.5) (layer "B.Cu") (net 11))
 (segment (start 167 48.62) (end 162.38 44) (width 0.5) (layer "B.Cu") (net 11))
 (segment (start 179.57 42.05) (end 174.49 42.05) (width 0.5) (layer "F.Cu") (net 9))
 (segment (start 180.57 54.77056) (end 180.57 43.05) (width 0.5) (layer "F.Cu") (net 9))
 (segment (start 180.57 43.05) (end 179.57 42.05) (width 0.5) (layer "F.Cu") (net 9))
 (segment (start 174.49 42.05) (end 172.54 44) (width 0.5) (layer "F.Cu") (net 9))
 (segment (start 163 72.07) (end 163.27056 72.07) (width 0.5) (layer "F.Cu") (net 9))
 (segment (start 163.27056 72.07) (end 180.57 54.77056) (width 0.5) (layer "F.Cu") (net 9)))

